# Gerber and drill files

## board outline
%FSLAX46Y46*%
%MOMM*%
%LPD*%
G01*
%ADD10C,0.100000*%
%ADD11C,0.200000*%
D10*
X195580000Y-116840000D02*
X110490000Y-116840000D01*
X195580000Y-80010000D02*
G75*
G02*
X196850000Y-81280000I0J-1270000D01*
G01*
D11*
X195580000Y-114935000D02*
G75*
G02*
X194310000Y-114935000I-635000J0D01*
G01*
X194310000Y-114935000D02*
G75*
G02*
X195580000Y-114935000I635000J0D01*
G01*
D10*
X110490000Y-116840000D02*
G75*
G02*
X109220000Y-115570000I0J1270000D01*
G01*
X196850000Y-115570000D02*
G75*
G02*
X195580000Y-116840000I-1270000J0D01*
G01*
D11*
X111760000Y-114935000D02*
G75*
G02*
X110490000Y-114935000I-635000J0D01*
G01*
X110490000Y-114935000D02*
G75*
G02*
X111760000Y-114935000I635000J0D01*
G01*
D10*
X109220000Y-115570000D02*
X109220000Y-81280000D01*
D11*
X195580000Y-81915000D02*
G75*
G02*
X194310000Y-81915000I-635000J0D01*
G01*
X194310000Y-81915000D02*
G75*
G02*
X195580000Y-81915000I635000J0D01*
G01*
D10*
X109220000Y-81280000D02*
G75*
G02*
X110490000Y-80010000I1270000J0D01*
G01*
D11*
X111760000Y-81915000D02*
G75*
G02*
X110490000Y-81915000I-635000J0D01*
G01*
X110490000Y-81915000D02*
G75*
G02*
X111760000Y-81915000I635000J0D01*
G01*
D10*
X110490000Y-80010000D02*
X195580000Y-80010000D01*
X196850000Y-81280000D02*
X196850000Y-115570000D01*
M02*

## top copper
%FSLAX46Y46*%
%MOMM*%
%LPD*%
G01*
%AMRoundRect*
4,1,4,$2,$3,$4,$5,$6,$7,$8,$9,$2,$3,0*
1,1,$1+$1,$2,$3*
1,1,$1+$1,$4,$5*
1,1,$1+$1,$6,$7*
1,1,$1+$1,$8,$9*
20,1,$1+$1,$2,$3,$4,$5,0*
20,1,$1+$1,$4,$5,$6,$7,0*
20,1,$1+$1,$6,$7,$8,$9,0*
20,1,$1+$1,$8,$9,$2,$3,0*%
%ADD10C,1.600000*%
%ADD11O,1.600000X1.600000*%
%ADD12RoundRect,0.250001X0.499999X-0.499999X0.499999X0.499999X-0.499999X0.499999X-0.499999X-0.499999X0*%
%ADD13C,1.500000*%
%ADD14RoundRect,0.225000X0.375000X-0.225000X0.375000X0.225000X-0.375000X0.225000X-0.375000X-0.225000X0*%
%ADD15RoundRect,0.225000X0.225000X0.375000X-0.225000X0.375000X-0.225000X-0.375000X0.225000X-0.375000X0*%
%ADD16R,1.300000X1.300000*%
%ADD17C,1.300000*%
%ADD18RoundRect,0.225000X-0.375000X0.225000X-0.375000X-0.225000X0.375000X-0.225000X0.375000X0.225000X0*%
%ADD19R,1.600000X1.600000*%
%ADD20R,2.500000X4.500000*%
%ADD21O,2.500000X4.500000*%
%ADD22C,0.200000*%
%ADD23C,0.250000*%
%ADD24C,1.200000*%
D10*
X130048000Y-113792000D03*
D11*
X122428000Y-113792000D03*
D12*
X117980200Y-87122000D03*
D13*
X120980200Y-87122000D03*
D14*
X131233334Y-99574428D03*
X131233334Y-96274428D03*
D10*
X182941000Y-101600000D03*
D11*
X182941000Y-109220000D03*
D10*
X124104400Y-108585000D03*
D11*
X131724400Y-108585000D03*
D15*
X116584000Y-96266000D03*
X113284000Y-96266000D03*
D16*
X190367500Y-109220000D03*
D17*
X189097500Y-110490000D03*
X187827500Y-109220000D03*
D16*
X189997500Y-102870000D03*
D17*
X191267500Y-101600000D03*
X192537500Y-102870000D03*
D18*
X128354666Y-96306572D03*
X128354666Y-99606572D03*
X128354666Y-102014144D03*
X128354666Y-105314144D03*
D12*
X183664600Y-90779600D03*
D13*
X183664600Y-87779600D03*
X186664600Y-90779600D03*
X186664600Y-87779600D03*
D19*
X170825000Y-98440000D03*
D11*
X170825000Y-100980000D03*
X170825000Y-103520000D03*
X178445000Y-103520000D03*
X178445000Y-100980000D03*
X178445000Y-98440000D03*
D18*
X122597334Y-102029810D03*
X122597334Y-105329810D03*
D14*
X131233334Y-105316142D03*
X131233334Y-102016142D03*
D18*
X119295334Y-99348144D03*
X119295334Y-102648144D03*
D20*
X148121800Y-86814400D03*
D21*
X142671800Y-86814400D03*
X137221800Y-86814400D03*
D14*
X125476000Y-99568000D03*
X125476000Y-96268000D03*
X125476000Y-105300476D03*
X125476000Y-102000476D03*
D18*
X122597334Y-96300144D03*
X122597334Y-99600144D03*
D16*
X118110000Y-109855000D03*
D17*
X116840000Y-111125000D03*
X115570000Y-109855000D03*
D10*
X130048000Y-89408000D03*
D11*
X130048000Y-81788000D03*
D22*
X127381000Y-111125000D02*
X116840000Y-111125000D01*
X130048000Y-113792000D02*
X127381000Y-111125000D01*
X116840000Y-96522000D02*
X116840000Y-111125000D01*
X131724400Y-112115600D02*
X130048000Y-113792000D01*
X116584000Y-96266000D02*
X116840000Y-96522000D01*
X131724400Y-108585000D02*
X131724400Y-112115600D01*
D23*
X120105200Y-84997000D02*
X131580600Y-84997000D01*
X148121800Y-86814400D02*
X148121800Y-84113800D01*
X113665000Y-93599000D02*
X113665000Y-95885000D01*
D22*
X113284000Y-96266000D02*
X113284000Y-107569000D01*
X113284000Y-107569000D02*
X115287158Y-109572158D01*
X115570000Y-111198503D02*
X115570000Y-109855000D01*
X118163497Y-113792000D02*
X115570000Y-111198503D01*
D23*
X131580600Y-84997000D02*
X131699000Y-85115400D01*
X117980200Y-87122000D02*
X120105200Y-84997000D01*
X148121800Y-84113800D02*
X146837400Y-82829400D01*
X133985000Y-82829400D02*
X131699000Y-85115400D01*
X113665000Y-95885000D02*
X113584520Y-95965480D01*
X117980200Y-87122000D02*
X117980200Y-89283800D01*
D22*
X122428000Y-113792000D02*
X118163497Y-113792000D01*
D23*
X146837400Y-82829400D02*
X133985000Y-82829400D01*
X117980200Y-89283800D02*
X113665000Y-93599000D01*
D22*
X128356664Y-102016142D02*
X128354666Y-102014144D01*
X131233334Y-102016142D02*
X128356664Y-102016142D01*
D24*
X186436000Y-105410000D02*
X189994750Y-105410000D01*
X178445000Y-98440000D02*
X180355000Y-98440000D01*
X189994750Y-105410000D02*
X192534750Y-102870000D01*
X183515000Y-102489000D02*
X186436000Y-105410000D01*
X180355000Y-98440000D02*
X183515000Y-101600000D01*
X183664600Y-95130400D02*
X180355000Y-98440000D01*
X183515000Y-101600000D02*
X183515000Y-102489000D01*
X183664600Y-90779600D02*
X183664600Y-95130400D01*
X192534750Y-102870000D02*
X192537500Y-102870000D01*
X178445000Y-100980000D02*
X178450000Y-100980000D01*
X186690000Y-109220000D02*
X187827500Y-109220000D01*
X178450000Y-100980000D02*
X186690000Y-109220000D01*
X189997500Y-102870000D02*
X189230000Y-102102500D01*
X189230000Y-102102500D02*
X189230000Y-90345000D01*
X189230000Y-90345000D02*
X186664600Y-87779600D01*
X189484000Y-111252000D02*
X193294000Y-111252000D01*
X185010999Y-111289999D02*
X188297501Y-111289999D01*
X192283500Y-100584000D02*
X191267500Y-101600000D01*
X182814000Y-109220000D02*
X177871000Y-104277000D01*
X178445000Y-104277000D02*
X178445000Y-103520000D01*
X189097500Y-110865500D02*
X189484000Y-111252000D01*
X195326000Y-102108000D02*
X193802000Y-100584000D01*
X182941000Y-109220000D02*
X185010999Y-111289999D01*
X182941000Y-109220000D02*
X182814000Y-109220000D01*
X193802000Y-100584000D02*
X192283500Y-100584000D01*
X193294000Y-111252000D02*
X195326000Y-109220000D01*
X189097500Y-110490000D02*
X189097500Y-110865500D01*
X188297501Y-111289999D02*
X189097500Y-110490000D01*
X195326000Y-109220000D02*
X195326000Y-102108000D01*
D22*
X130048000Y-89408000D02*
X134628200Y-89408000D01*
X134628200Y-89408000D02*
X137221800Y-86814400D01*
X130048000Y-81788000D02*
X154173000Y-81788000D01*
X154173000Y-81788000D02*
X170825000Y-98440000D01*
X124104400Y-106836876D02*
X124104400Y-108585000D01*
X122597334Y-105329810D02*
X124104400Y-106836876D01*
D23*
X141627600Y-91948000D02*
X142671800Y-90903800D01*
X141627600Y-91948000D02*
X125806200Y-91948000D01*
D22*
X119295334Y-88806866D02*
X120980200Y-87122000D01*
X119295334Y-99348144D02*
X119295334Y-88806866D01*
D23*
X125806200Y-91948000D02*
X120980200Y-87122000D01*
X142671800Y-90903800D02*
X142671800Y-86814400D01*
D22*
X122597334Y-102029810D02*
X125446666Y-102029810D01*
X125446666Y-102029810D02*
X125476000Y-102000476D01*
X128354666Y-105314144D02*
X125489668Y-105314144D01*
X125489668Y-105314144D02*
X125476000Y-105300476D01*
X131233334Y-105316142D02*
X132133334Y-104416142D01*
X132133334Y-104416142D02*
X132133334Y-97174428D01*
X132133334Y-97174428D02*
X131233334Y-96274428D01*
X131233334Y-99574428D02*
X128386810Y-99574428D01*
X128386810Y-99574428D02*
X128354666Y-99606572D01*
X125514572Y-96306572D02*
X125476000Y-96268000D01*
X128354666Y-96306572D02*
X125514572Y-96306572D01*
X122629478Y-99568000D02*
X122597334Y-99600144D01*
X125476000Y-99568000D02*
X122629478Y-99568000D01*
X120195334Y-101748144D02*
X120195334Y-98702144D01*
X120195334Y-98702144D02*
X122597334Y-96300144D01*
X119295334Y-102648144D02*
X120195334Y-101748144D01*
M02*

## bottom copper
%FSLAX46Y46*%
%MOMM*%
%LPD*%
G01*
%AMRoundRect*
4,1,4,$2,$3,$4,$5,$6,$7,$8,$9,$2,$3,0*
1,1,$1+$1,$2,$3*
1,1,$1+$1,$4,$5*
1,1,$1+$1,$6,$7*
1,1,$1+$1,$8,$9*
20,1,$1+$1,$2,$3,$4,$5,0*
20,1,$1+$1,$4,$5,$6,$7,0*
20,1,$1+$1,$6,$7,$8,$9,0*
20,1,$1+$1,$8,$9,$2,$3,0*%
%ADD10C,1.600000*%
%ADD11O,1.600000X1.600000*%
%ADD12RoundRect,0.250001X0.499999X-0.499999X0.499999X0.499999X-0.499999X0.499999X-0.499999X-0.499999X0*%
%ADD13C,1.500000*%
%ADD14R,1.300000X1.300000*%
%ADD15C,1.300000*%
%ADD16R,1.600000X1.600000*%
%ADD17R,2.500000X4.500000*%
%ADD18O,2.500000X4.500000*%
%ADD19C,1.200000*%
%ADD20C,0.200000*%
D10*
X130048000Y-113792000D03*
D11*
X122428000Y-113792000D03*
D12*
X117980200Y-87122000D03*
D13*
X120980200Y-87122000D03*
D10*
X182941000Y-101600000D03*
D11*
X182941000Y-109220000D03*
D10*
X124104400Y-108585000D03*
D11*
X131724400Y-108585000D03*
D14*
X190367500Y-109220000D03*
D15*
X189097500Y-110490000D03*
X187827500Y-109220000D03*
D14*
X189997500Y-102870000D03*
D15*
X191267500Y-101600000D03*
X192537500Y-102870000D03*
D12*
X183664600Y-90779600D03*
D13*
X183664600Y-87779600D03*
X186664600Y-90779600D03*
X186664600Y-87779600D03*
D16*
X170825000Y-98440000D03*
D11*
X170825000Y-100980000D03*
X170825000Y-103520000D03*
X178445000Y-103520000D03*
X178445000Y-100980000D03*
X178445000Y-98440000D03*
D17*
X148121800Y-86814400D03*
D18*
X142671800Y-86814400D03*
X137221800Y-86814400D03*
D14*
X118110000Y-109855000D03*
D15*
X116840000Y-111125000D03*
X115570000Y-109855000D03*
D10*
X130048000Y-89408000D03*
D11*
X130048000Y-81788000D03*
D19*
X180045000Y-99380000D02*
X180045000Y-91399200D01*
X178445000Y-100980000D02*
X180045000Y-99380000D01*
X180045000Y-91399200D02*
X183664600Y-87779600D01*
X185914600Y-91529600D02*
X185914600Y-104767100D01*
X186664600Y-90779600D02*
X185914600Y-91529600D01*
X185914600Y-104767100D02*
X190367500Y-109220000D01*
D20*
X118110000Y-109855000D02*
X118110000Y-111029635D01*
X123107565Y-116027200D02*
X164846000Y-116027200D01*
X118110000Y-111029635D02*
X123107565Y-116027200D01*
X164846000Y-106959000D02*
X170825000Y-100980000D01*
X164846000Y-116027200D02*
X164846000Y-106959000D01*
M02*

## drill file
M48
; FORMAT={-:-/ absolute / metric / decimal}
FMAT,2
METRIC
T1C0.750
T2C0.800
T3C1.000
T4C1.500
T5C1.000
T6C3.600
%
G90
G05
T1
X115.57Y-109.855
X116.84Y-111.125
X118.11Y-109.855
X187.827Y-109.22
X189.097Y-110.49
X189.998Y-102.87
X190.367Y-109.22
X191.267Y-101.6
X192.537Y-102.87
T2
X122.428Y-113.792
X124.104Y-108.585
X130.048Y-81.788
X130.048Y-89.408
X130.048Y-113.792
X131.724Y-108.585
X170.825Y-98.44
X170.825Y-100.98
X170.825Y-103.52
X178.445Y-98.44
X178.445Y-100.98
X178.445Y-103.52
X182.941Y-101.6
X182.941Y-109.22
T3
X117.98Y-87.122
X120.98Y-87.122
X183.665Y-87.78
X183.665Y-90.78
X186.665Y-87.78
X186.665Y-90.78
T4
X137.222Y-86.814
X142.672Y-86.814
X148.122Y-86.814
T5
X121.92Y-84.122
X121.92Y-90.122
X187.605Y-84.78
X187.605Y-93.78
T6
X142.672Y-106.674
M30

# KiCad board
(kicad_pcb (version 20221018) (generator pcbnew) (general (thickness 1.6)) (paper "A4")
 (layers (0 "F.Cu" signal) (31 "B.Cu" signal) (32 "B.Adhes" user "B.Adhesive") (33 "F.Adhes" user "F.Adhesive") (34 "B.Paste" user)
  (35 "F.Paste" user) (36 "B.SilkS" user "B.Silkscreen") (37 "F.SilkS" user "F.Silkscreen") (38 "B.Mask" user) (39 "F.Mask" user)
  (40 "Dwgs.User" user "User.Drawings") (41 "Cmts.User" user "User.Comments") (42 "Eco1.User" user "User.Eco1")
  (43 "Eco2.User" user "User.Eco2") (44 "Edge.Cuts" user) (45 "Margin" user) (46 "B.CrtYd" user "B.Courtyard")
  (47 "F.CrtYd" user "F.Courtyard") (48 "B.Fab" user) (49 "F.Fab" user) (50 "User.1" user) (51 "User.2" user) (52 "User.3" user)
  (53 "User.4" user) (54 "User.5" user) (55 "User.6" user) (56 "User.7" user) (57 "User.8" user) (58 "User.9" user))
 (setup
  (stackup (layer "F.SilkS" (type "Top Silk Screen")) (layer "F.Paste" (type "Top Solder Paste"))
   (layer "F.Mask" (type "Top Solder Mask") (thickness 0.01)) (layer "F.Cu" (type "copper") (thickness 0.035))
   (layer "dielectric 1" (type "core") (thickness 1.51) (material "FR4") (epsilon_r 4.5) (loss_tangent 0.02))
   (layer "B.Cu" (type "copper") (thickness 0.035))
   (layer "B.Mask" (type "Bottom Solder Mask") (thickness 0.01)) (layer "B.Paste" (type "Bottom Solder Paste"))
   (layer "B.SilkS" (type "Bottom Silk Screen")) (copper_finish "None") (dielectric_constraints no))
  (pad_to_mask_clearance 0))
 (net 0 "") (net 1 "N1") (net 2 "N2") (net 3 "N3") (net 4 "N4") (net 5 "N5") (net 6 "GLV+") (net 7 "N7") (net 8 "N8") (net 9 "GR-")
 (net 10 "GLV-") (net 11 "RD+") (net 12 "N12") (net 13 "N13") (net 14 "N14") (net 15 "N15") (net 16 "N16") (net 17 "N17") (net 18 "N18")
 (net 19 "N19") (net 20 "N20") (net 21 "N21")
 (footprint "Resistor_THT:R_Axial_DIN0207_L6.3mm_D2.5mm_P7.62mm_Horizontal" (layer "F.Cu") (at 130.048 113.792 180)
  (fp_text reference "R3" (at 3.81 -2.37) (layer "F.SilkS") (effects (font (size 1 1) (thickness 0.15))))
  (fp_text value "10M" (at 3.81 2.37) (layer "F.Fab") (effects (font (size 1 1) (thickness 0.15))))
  (pad "1" thru_hole circle (at 0 0 180) (size 1.6 1.6) (drill 0.8) (layers "*.Cu" "*.Mask") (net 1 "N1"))
  (pad "2" thru_hole oval (at 7.62 0 180) (size 1.6 1.6) (drill 0.8) (layers "*.Cu" "*.Mask") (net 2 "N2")))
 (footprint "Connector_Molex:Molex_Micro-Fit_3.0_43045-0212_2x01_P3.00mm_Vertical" (layer "F.Cu") (at 117.9802 87.122 90)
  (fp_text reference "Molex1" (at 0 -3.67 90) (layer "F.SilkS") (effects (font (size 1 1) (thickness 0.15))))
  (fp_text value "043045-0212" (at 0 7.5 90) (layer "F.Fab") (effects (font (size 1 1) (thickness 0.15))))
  (pad "" np_thru_hole circle (at -3 3.94 90) (size 1 1) (drill 1) (layers "*.Cu" "*.Mask"))
  (pad "" np_thru_hole circle (at 3 3.94 90) (size 1 1) (drill 1) (layers "*.Cu" "*.Mask"))
  (pad "1" thru_hole roundrect (at 0 0 90) (size 1.5 1.5) (drill 1) (layers "*.Cu" "*.Mask") (roundrect_rratio 0.166667) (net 2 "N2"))
  (pad "2" thru_hole circle (at 0 3 90) (size 1.5 1.5) (drill 1) (layers "*.Cu" "*.Mask") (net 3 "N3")))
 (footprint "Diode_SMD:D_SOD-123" (layer "F.Cu") (at 131.233334 97.924428 90)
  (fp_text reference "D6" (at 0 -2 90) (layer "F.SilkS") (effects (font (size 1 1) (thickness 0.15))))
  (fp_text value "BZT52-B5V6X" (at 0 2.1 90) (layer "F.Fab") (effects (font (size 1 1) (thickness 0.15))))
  (pad "1" smd roundrect (at -1.65 0 90) (size 0.9 1.2) (layers "F.Cu" "F.Paste" "F.Mask") (roundrect_rratio 0.25) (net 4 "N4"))
  (pad "2" smd roundrect (at 1.65 0 90) (size 0.9 1.2) (layers "F.Cu" "F.Paste" "F.Mask") (roundrect_rratio 0.25) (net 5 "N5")))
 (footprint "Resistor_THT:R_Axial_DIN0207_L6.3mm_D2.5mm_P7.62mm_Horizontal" (layer "F.Cu") (at 182.941 101.6 -90)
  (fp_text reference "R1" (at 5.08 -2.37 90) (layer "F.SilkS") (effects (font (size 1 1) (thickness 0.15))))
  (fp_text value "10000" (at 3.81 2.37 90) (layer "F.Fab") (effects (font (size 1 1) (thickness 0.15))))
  (pad "1" thru_hole circle (at 0 0 270) (size 1.6 1.6) (drill 0.8) (layers "*.Cu" "*.Mask") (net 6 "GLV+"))
  (pad "2" thru_hole oval (at 7.62 0 270) (size 1.6 1.6) (drill 0.8) (layers "*.Cu" "*.Mask") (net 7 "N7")))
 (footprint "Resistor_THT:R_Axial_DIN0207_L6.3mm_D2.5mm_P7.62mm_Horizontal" (layer "F.Cu") (at 124.1044 108.585)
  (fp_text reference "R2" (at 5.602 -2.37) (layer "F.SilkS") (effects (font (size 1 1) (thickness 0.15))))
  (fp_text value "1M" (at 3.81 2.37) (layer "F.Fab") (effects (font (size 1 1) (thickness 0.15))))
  (pad "1" thru_hole circle (at 0 0) (size 1.6 1.6) (drill 0.8) (layers "*.Cu" "*.Mask") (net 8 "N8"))
  (pad "2" thru_hole oval (at 7.62 0) (size 1.6 1.6) (drill 0.8) (layers "*.Cu" "*.Mask") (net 1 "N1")))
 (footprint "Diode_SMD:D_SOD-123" (layer "F.Cu") (at 114.934 96.266 180)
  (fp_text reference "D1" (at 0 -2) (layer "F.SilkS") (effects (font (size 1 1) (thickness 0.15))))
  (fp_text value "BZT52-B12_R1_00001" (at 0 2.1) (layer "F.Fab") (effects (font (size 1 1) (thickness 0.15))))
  (pad "1" smd roundrect (at -1.65 0 180) (size 0.9 1.2) (layers "F.Cu" "F.Paste" "F.Mask") (roundrect_rratio 0.25) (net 1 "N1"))
  (pad "2" smd roundrect (at 1.65 0 180) (size 0.9 1.2) (layers "F.Cu" "F.Paste" "F.Mask") (roundrect_rratio 0.25) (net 2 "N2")))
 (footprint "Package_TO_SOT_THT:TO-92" (layer "F.Cu") (at 190.3675 109.22 180)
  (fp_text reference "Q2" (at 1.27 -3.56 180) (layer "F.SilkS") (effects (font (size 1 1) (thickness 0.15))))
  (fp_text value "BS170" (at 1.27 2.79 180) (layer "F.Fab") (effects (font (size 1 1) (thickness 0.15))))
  (pad "1" thru_hole rect (at 0 0 180) (size 1.3 1.3) (drill 0.75) (layers "*.Cu" "*.Mask") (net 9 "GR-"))
  (pad "2" thru_hole circle (at 1.27 -1.27 180) (size 1.3 1.3) (drill 0.75) (layers "*.Cu" "*.Mask") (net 7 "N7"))
  (pad "3" thru_hole circle (at 2.54 0 180) (size 1.3 1.3) (drill 0.75) (layers "*.Cu" "*.Mask") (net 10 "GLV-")))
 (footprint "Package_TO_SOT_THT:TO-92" (layer "F.Cu") (at 189.9975 102.87)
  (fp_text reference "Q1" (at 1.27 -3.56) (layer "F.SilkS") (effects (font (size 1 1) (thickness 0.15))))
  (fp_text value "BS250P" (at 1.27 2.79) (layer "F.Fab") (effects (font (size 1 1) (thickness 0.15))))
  (pad "1" thru_hole rect (at 0 0) (size 1.3 1.3) (drill 0.75) (layers "*.Cu" "*.Mask") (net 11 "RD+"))
  (pad "2" thru_hole circle (at 1.27 -1.27) (size 1.3 1.3) (drill 0.75) (layers "*.Cu" "*.Mask") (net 7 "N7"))
  (pad "3" thru_hole circle (at 2.54 0) (size 1.3 1.3) (drill 0.75) (layers "*.Cu" "*.Mask") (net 6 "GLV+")))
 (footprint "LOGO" (layer "F.Cu") (at 157.988 103.124)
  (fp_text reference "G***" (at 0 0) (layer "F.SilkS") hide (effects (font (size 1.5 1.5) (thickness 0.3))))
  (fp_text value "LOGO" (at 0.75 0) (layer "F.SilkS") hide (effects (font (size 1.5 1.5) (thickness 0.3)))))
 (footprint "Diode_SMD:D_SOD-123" (layer "F.Cu") (at 128.354666 97.956572 -90)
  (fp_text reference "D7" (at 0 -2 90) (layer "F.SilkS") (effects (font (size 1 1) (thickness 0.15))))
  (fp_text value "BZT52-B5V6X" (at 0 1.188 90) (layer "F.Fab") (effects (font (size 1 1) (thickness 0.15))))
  (pad "1" smd roundrect (at -1.65 0 270) (size 0.9 1.2) (layers "F.Cu" "F.Paste" "F.Mask") (roundrect_rratio 0.25) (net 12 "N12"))
  (pad "2" smd roundrect (at 1.65 0 270) (size 0.9 1.2) (layers "F.Cu" "F.Paste" "F.Mask") (roundrect_rratio 0.25) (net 4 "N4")))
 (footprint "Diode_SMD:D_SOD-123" (layer "F.Cu") (at 128.354666 103.664144 -90)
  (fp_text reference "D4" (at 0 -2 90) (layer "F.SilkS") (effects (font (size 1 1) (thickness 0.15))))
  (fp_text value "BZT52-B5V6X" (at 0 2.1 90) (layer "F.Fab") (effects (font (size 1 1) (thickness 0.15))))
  (pad "1" smd roundrect (at -1.65 0 270) (size 0.9 1.2) (layers "F.Cu" "F.Paste" "F.Mask") (roundrect_rratio 0.25) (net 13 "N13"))
  (pad "2" smd roundrect (at 1.65 0 270) (size 0.9 1.2) (layers "F.Cu" "F.Paste" "F.Mask") (roundrect_rratio 0.25) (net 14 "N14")))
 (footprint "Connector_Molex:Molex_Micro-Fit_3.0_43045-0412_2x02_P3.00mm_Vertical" (layer "F.Cu") (at 183.6646 90.7796 90)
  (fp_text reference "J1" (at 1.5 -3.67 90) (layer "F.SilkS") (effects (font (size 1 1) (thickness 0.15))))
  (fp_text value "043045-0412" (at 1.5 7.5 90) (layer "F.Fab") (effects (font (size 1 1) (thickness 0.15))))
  (pad "" np_thru_hole circle (at -3 3.94 90) (size 1 1) (drill 1) (layers "*.Cu" "*.Mask"))
  (pad "" np_thru_hole circle (at 6 3.94 90) (size 1 1) (drill 1) (layers "*.Cu" "*.Mask"))
  (pad "1" thru_hole roundrect (at 0 0 90) (size 1.5 1.5) (drill 1) (layers "*.Cu" "*.Mask") (roundrect_rratio 0.166667) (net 6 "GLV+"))
  (pad "2" thru_hole circle (at 3 0 90) (size 1.5 1.5) (drill 1) (layers "*.Cu" "*.Mask") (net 10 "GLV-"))
  (pad "3" thru_hole circle (at 0 3 90) (size 1.5 1.5) (drill 1) (layers "*.Cu" "*.Mask") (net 9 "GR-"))
  (pad "4" thru_hole circle (at 3 3 90) (size 1.5 1.5) (drill 1) (layers "*.Cu" "*.Mask") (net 11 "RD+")))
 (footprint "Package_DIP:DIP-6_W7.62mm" (layer "F.Cu") (at 170.825 98.44)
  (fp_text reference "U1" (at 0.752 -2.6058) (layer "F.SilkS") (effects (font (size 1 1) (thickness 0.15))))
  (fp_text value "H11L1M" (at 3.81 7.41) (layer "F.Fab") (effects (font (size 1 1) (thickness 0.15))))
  (pad "1" thru_hole rect (at 0 0) (size 1.6 1.6) (drill 0.8) (layers "*.Cu" "*.Mask") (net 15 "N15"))
  (pad "2" thru_hole oval (at 0 2.54) (size 1.6 1.6) (drill 0.8) (layers "*.Cu" "*.Mask") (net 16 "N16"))
  (pad "3" thru_hole oval (at 0 5.08) (size 1.6 1.6) (drill 0.8) (layers "*.Cu" "*.Mask") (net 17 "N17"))
  (pad "4" thru_hole oval (at 7.62 5.08) (size 1.6 1.6) (drill 0.8) (layers "*.Cu" "*.Mask") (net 7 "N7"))
  (pad "5" thru_hole oval (at 7.62 2.54) (size 1.6 1.6) (drill 0.8) (layers "*.Cu" "*.Mask") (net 10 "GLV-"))
  (pad "6" thru_hole oval (at 7.62 0) (size 1.6 1.6) (drill 0.8) (layers "*.Cu" "*.Mask") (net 6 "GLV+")))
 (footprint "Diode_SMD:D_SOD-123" (layer "F.Cu") (at 122.597334 103.67981 -90)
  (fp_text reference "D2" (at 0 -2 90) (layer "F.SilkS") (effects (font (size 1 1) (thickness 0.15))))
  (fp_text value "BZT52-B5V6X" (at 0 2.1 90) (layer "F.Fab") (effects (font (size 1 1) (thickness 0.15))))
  (pad "1" smd roundrect (at -1.65 0 270) (size 0.9 1.2) (layers "F.Cu" "F.Paste" "F.Mask") (roundrect_rratio 0.25) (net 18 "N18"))
  (pad "2" smd roundrect (at 1.65 0 270) (size 0.9 1.2) (layers "F.Cu" "F.Paste" "F.Mask") (roundrect_rratio 0.25) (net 8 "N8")))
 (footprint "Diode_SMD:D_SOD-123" (layer "F.Cu") (at 131.233334 103.666142 90)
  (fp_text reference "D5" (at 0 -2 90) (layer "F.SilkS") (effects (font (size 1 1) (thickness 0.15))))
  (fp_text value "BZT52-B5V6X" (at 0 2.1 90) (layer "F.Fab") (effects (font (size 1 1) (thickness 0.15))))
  (pad "1" smd roundrect (at -1.65 0 90) (size 0.9 1.2) (layers "F.Cu" "F.Paste" "F.Mask") (roundrect_rratio 0.25) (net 5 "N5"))
  (pad "2" smd roundrect (at 1.65 0 90) (size 0.9 1.2) (layers "F.Cu" "F.Paste" "F.Mask") (roundrect_rratio 0.25) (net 13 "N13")))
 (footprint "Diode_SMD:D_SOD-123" (layer "F.Cu") (at 119.295334 100.998144 -90)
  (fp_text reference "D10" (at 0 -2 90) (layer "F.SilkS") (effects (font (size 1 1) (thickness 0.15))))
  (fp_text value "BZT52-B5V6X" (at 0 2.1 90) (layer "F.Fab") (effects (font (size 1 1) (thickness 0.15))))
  (pad "1" smd roundrect (at -1.65 0 270) (size 0.9 1.2) (layers "F.Cu" "F.Paste" "F.Mask") (roundrect_rratio 0.25) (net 3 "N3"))
  (pad "2" smd roundrect (at 1.65 0 270) (size 0.9 1.2) (layers "F.Cu" "F.Paste" "F.Mask") (roundrect_rratio 0.25) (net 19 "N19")))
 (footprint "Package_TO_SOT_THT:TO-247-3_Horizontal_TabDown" (layer "F.Cu") (at 148.1218 86.8144 180)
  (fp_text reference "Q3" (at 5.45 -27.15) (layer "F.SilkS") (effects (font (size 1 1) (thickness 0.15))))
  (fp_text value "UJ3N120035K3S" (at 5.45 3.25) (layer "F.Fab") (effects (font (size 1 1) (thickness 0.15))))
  (pad "" np_thru_hole oval (at 5.45 -19.86 180) (size 3.6 3.6) (drill 3.6) (layers "*.Cu" "*.Mask"))
  (pad "1" thru_hole rect (at 0 0 180) (size 2.5 4.5) (drill 1.5) (layers "*.Cu" "*.Mask") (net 2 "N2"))
  (pad "2" thru_hole oval (at 5.45 0 180) (size 2.5 4.5) (drill 1.5) (layers "*.Cu" "*.Mask") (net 3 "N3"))
  (pad "3" thru_hole oval (at 10.9 0 180) (size 2.5 4.5) (drill 1.5) (layers "*.Cu" "*.Mask") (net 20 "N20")))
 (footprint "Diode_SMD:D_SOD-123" (layer "F.Cu") (at 125.476 97.918 90)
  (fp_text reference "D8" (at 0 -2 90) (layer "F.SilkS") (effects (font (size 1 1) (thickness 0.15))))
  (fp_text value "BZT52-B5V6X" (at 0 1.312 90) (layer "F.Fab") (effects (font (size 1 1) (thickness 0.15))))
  (pad "1" smd roundrect (at -1.65 0 90) (size 0.9 1.2) (layers "F.Cu" "F.Paste" "F.Mask") (roundrect_rratio 0.25) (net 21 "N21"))
  (pad "2" smd roundrect (at 1.65 0 90) (size 0.9 1.2) (layers "F.Cu" "F.Paste" "F.Mask") (roundrect_rratio 0.25) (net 12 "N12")))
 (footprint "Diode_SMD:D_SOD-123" (layer "F.Cu") (at 125.476 103.650476 90)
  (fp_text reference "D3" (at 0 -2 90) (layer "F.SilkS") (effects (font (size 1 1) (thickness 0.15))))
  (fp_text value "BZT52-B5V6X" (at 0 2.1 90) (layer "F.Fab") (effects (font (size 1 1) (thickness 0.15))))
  (pad "1" smd roundrect (at -1.65 0 90) (size 0.9 1.2) (layers "F.Cu" "F.Paste" "F.Mask") (roundrect_rratio 0.25) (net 14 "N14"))
  (pad "2" smd roundrect (at 1.65 0 90) (size 0.9 1.2) (layers "F.Cu" "F.Paste" "F.Mask") (roundrect_rratio 0.25) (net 18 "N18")))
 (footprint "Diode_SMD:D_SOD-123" (layer "F.Cu") (at 122.597334 97.950144 -90)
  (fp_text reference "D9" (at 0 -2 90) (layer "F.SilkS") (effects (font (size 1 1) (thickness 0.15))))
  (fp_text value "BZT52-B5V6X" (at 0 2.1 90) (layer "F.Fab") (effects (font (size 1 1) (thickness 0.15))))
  (pad "1" smd roundrect (at -1.65 0 270) (size 0.9 1.2) (layers "F.Cu" "F.Paste" "F.Mask") (roundrect_rratio 0.25) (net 19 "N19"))
  (pad "2" smd roundrect (at 1.65 0 270) (size 0.9 1.2) (layers "F.Cu" "F.Paste" "F.Mask") (roundrect_rratio 0.25) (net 21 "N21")))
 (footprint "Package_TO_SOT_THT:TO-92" (layer "F.Cu") (at 118.11 109.855 180)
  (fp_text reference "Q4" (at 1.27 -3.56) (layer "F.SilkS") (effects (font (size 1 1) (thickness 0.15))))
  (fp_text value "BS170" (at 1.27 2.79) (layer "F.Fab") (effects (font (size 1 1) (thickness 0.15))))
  (pad "1" thru_hole rect (at 0 0 180) (size 1.3 1.3) (drill 0.75) (layers "*.Cu" "*.Mask") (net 16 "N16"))
  (pad "2" thru_hole circle (at 1.27 -1.27 180) (size 1.3 1.3) (drill 0.75) (layers "*.Cu" "*.Mask") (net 1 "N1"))
  (pad "3" thru_hole circle (at 2.54 0 180) (size 1.3 1.3) (drill 0.75) (layers "*.Cu" "*.Mask") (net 2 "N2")))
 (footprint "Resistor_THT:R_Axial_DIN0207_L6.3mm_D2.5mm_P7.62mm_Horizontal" (layer "F.Cu") (at 130.048 89.408 90)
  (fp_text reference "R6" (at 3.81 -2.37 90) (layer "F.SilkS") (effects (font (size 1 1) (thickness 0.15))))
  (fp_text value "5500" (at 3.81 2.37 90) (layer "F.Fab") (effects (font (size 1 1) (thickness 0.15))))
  (pad "1" thru_hole circle (at 0 0 90) (size 1.6 1.6) (drill 0.8) (layers "*.Cu" "*.Mask") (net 20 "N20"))
  (pad "2" thru_hole oval (at 7.62 0 90) (size 1.6 1.6) (drill 0.8) (layers "*.Cu" "*.Mask") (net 15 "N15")))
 (gr_line (start 195.58 116.84) (end 110.49 116.84) (stroke (width 0.1) (type default)) (layer "Edge.Cuts"))
 (gr_arc (start 195.58 80.01) (mid 196.478026 80.381974) (end 196.85 81.28) (stroke (width 0.1) (type default)) (layer "Edge.Cuts"))
 (gr_circle (center 194.945 114.935) (end 195.58 114.935) (stroke (width 0.2) (type default)) (fill none) (layer "Edge.Cuts"))
 (gr_arc (start 110.49 116.84) (mid 109.591974 116.468026) (end 109.22 115.57) (stroke (width 0.1) (type default)) (layer "Edge.Cuts"))
 (gr_arc (start 196.85 115.57) (mid 196.478026 116.468026) (end 195.58 116.84) (stroke (width 0.1) (type default)) (layer "Edge.Cuts"))
 (gr_circle (center 111.125 114.935) (end 111.76 114.935) (stroke (width 0.2) (type default)) (fill none) (layer "Edge.Cuts"))
 (gr_line (start 109.22 115.57) (end 109.22 81.28) (stroke (width 0.1) (type default)) (layer "Edge.Cuts"))
 (gr_circle (center 194.945 81.915) (end 195.58 81.915) (stroke (width 0.2) (type default)) (fill none) (layer "Edge.Cuts"))
 (gr_arc (start 109.22 81.28) (mid 109.591974 80.381974) (end 110.49 80.01) (stroke (width 0.1) (type default)) (layer "Edge.Cuts"))
 (gr_circle (center 111.125 81.915) (end 111.76 81.915) (stroke (width 0.2) (type default)) (fill none) (layer "Edge.Cuts"))
 (gr_line (start 110.49 80.01) (end 195.58 80.01) (stroke (width 0.1) (type default)) (layer "Edge.Cuts"))
 (gr_line (start 196.85 81.28) (end 196.85 115.57) (stroke (width 0.1) (type default)) (layer "Edge.Cuts"))
 (segment (start 127.381 111.125) (end 116.84 111.125) (width 0.2) (layer "F.Cu") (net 1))
 (segment (start 130.048 113.792) (end 127.381 111.125) (width 0.2) (layer "F.Cu") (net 1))
 (segment (start 116.84 96.522) (end 116.84 111.125) (width 0.2) (layer "F.Cu") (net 1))
 (segment (start 131.7244 112.1156) (end 130.048 113.792) (width 0.2) (layer "F.Cu") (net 1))
 (segment (start 116.584 96.266) (end 116.84 96.522) (width 0.2) (layer "F.Cu") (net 1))
 (segment (start 131.7244 108.585) (end 131.7244 112.1156) (width 0.2) (layer "F.Cu") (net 1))
 (segment (start 120.1052 84.997) (end 131.5806 84.997) (width 0.25) (layer "F.Cu") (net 2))
 (segment (start 148.1218 86.8144) (end 148.1218 84.1138) (width 0.25) (layer "F.Cu") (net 2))
 (segment (start 113.665 93.599) (end 113.665 95.885) (width 0.25) (layer "F.Cu") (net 2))
 (segment (start 113.284 96.266) (end 113.284 107.569) (width 0.2) (layer "F.Cu") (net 2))
 (segment (start 113.284 107.569) (end 115.287158 109.572158) (width 0.2) (layer "F.Cu") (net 2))
 (segment (start 115.57 111.198503) (end 115.57 109.855) (width 0.2) (layer "F.Cu") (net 2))
 (segment (start 118.163497 113.792) (end 115.57 111.198503) (width 0.2) (layer "F.Cu") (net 2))
 (segment (start 131.5806 84.997) (end 131.699 85.1154) (width 0.25) (layer "F.Cu") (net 2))
 (segment (start 117.9802 87.122) (end 120.1052 84.997) (width 0.25) (layer "F.Cu") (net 2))
 (segment (start 148.1218 84.1138) (end 146.8374 82.8294) (width 0.25) (layer "F.Cu") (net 2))
 (segment (start 133.985 82.8294) (end 131.699 85.1154) (width 0.25) (layer "F.Cu") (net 2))
 (segment (start 113.665 95.885) (end 113.58452 95.96548) (width 0.25) (layer "F.Cu") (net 2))
 (segment (start 117.9802 87.122) (end 117.9802 89.2838) (width 0.25) (layer "F.Cu") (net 2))
 (segment (start 122.428 113.792) (end 118.163497 113.792) (width 0.2) (layer "F.Cu") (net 2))
 (segment (start 146.8374 82.8294) (end 133.985 82.8294) (width 0.25) (layer "F.Cu") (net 2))
 (segment (start 117.9802 89.2838) (end 113.665 93.599) (width 0.25) (layer "F.Cu") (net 2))
 (segment (start 128.356664 102.016142) (end 128.354666 102.014144) (width 0.2) (layer "F.Cu") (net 13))
 (segment (start 131.233334 102.016142) (end 128.356664 102.016142) (width 0.2) (layer "F.Cu") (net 13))
 (segment (start 186.436 105.41) (end 189.99475 105.41) (width 1.2) (layer "F.Cu") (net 6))
 (segment (start 178.445 98.44) (end 180.355 98.44) (width 1.2) (layer "F.Cu") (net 6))
 (segment (start 189.99475 105.41) (end 192.53475 102.87) (width 1.2) (layer "F.Cu") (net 6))
 (segment (start 183.515 102.489) (end 186.436 105.41) (width 1.2) (layer "F.Cu") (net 6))
 (segment (start 180.355 98.44) (end 183.515 101.6) (width 1.2) (layer "F.Cu") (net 6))
 (segment (start 183.6646 95.1304) (end 180.355 98.44) (width 1.2) (layer "F.Cu") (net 6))
 (segment (start 183.515 101.6) (end 183.515 102.489) (width 1.2) (layer "F.Cu") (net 6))
 (segment (start 183.6646 90.7796) (end 183.6646 95.1304) (width 1.2) (layer "F.Cu") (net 6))
 (segment (start 192.53475 102.87) (end 192.5375 102.87) (width 1.2) (layer "F.Cu") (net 6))
 (segment (start 178.445 100.98) (end 178.45 100.98) (width 1.2) (layer "F.Cu") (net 10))
 (segment (start 186.69 109.22) (end 187.8275 109.22) (width 1.2) (layer "F.Cu") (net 10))
 (segment (start 178.45 100.98) (end 186.69 109.22) (width 1.2) (layer "F.Cu") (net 10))
 (segment (start 180.045 99.38) (end 180.045 91.3992) (width 1.2) (layer "B.Cu") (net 10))
 (segment (start 178.445 100.98) (end 180.045 99.38) (width 1.2) (layer "B.Cu") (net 10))
 (segment (start 180.045 91.3992) (end 183.6646 87.7796) (width 1.2) (layer "B.Cu") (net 10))
 (segment (start 185.9146 91.5296) (end 185.9146 104.7671) (width 1.2) (layer "B.Cu") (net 9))
 (segment (start 186.6646 90.7796) (end 185.9146 91.5296) (width 1.2) (layer "B.Cu") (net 9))
 (segment (start 185.9146 104.7671) (end 190.3675 109.22) (width 1.2) (layer "B.Cu") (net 9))
 (segment (start 189.9975 102.87) (end 189.23 102.1025) (width 1.2) (layer "F.Cu") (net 11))
 (segment (start 189.23 102.1025) (end 189.23 90.345) (width 1.2) (layer "F.Cu") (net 11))
 (segment (start 189.23 90.345) (end 186.6646 87.7796) (width 1.2) (layer "F.Cu") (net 11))
 (segment (start 189.484 111.252) (end 193.294 111.252) (width 1.2) (layer "F.Cu") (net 7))
 (segment (start 185.010999 111.289999) (end 188.297501 111.289999) (width 1.2) (layer "F.Cu") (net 7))
 (segment (start 192.2835 100.584) (end 191.2675 101.6) (width 1.2) (layer "F.Cu") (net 7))
 (segment (start 182.814 109.22) (end 177.871 104.277) (width 1.2) (layer "F.Cu") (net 7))
 (segment (start 178.445 104.277) (end 178.445 103.52) (width 1.2) (layer "F.Cu") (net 7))
 (segment (start 189.0975 110.8655) (end 189.484 111.252) (width 1.2) (layer "F.Cu") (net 7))
 (segment (start 195.326 102.108) (end 193.802 100.584) (width 1.2) (layer "F.Cu") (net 7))
 (segment (start 182.941 109.22) (end 185.010999 111.289999) (width 1.2) (layer "F.Cu") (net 7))
 (segment (start 182.941 109.22) (end 182.814 109.22) (width 1.2) (layer "F.Cu") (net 7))
 (segment (start 193.802 100.584) (end 192.2835 100.584) (width 1.2) (layer "F.Cu") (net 7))
 (segment (start 193.294 111.252) (end 195.326 109.22) (width 1.2) (layer "F.Cu") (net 7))
 (segment (start 189.0975 110.49) (end 189.0975 110.8655) (width 1.2) (layer "F.Cu") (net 7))
 (segment (start 188.297501 111.289999) (end 189.0975 110.49) (width 1.2) (layer "F.Cu") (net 7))
 (segment (start 195.326 109.22) (end 195.326 102.108) (width 1.2) (layer "F.Cu") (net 7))
 (segment (start 130.048 89.408) (end 134.6282 89.408) (width 0.2) (layer "F.Cu") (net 20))
 (segment (start 134.6282 89.408) (end 137.2218 86.8144) (width 0.2) (layer "F.Cu") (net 20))
 (segment (start 118.11 109.855) (end 118.11 111.029635) (width 0.2) (layer "B.Cu") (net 16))
 (segment (start 123.107565 116.0272) (end 164.846 116.0272) (width 0.2) (layer "B.Cu") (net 16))
 (segment (start 118.11 111.029635) (end 123.107565 116.0272) (width 0.2) (layer "B.Cu") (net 16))
 (segment (start 164.846 106.959) (end 170.825 100.98) (width 0.2) (layer "B.Cu") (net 16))
 (segment (start 164.846 116.0272) (end 164.846 106.959) (width 0.2) (layer "B.Cu") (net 16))
 (segment (start 130.048 81.788) (end 154.173 81.788) (width 0.2) (layer "F.Cu") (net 15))
 (segment (start 154.173 81.788) (end 170.825 98.44) (width 0.2) (layer "F.Cu") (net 15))
 (segment (start 124.1044 106.836876) (end 124.1044 108.585) (width 0.2) (layer "F.Cu") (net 8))
 (segment (start 122.597334 105.32981) (end 124.1044 106.836876) (width 0.2) (layer "F.Cu") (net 8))
 (segment (start 141.6276 91.948) (end 142.6718 90.9038) (width 0.25) (layer "F.Cu") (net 3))
 (segment (start 141.6276 91.948) (end 125.8062 91.948) (width 0.25) (layer "F.Cu") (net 3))
 (segment (start 119.295334 88.806866) (end 120.9802 87.122) (width 0.2) (layer "F.Cu") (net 3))
 (segment (start 119.295334 99.348144) (end 119.295334 88.806866) (width 0.2) (layer "F.Cu") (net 3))
 (segment (start 125.8062 91.948) (end 120.9802 87.122) (width 0.25) (layer "F.Cu") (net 3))
 (segment (start 142.6718 90.9038) (end 142.6718 86.8144) (width 0.25) (layer "F.Cu") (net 3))
 (segment (start 122.597334 102.02981) (end 125.446666 102.02981) (width 0.2) (layer "F.Cu") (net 18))
 (segment (start 125.446666 102.02981) (end 125.476 102.000476) (width 0.2) (layer "F.Cu") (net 18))
 (segment (start 128.354666 105.314144) (end 125.489668 105.314144) (width 0.2) (layer "F.Cu") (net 14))
 (segment (start 125.489668 105.314144) (end 125.476 105.300476) (width 0.2) (layer "F.Cu") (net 14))
 (segment (start 131.233334 105.316142) (end 132.133334 104.416142) (width 0.2) (layer "F.Cu") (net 5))
 (segment (start 132.133334 104.416142) (end 132.133334 97.174428) (width 0.2) (layer "F.Cu") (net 5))
 (segment (start 132.133334 97.174428) (end 131.233334 96.274428) (width 0.2) (layer "F.Cu") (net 5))
 (segment (start 131.233334 99.574428) (end 128.38681 99.574428) (width 0.2) (layer "F.Cu") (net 4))
 (segment (start 128.38681 99.574428) (end 128.354666 99.606572) (width 0.2) (layer "F.Cu") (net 4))
 (segment (start 125.514572 96.306572) (end 125.476 96.268) (width 0.2) (layer "F.Cu") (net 12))
 (segment (start 128.354666 96.306572) (end 125.514572 96.306572) (width 0.2) (layer "F.Cu") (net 12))
 (segment (start 122.629478 99.568) (end 122.597334 99.600144) (width 0.2) (layer "F.Cu") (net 21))
 (segment (start 125.476 99.568) (end 122.629478 99.568) (width 0.2) (layer "F.Cu") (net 21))
 (segment (start 120.195334 101.748144) (end 120.195334 98.702144) (width 0.2) (layer "F.Cu") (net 19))
 (segment (start 120.195334 98.702144) (end 122.597334 96.300144) (width 0.2) (layer "F.Cu") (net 19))
 (segment (start 119.295334 102.648144) (end 120.195334 101.748144) (width 0.2) (layer "F.Cu") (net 19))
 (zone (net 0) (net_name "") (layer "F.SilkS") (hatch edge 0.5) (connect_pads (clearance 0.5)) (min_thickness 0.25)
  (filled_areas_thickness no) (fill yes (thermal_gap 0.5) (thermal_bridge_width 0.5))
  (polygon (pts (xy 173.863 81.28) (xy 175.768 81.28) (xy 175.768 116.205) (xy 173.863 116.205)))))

